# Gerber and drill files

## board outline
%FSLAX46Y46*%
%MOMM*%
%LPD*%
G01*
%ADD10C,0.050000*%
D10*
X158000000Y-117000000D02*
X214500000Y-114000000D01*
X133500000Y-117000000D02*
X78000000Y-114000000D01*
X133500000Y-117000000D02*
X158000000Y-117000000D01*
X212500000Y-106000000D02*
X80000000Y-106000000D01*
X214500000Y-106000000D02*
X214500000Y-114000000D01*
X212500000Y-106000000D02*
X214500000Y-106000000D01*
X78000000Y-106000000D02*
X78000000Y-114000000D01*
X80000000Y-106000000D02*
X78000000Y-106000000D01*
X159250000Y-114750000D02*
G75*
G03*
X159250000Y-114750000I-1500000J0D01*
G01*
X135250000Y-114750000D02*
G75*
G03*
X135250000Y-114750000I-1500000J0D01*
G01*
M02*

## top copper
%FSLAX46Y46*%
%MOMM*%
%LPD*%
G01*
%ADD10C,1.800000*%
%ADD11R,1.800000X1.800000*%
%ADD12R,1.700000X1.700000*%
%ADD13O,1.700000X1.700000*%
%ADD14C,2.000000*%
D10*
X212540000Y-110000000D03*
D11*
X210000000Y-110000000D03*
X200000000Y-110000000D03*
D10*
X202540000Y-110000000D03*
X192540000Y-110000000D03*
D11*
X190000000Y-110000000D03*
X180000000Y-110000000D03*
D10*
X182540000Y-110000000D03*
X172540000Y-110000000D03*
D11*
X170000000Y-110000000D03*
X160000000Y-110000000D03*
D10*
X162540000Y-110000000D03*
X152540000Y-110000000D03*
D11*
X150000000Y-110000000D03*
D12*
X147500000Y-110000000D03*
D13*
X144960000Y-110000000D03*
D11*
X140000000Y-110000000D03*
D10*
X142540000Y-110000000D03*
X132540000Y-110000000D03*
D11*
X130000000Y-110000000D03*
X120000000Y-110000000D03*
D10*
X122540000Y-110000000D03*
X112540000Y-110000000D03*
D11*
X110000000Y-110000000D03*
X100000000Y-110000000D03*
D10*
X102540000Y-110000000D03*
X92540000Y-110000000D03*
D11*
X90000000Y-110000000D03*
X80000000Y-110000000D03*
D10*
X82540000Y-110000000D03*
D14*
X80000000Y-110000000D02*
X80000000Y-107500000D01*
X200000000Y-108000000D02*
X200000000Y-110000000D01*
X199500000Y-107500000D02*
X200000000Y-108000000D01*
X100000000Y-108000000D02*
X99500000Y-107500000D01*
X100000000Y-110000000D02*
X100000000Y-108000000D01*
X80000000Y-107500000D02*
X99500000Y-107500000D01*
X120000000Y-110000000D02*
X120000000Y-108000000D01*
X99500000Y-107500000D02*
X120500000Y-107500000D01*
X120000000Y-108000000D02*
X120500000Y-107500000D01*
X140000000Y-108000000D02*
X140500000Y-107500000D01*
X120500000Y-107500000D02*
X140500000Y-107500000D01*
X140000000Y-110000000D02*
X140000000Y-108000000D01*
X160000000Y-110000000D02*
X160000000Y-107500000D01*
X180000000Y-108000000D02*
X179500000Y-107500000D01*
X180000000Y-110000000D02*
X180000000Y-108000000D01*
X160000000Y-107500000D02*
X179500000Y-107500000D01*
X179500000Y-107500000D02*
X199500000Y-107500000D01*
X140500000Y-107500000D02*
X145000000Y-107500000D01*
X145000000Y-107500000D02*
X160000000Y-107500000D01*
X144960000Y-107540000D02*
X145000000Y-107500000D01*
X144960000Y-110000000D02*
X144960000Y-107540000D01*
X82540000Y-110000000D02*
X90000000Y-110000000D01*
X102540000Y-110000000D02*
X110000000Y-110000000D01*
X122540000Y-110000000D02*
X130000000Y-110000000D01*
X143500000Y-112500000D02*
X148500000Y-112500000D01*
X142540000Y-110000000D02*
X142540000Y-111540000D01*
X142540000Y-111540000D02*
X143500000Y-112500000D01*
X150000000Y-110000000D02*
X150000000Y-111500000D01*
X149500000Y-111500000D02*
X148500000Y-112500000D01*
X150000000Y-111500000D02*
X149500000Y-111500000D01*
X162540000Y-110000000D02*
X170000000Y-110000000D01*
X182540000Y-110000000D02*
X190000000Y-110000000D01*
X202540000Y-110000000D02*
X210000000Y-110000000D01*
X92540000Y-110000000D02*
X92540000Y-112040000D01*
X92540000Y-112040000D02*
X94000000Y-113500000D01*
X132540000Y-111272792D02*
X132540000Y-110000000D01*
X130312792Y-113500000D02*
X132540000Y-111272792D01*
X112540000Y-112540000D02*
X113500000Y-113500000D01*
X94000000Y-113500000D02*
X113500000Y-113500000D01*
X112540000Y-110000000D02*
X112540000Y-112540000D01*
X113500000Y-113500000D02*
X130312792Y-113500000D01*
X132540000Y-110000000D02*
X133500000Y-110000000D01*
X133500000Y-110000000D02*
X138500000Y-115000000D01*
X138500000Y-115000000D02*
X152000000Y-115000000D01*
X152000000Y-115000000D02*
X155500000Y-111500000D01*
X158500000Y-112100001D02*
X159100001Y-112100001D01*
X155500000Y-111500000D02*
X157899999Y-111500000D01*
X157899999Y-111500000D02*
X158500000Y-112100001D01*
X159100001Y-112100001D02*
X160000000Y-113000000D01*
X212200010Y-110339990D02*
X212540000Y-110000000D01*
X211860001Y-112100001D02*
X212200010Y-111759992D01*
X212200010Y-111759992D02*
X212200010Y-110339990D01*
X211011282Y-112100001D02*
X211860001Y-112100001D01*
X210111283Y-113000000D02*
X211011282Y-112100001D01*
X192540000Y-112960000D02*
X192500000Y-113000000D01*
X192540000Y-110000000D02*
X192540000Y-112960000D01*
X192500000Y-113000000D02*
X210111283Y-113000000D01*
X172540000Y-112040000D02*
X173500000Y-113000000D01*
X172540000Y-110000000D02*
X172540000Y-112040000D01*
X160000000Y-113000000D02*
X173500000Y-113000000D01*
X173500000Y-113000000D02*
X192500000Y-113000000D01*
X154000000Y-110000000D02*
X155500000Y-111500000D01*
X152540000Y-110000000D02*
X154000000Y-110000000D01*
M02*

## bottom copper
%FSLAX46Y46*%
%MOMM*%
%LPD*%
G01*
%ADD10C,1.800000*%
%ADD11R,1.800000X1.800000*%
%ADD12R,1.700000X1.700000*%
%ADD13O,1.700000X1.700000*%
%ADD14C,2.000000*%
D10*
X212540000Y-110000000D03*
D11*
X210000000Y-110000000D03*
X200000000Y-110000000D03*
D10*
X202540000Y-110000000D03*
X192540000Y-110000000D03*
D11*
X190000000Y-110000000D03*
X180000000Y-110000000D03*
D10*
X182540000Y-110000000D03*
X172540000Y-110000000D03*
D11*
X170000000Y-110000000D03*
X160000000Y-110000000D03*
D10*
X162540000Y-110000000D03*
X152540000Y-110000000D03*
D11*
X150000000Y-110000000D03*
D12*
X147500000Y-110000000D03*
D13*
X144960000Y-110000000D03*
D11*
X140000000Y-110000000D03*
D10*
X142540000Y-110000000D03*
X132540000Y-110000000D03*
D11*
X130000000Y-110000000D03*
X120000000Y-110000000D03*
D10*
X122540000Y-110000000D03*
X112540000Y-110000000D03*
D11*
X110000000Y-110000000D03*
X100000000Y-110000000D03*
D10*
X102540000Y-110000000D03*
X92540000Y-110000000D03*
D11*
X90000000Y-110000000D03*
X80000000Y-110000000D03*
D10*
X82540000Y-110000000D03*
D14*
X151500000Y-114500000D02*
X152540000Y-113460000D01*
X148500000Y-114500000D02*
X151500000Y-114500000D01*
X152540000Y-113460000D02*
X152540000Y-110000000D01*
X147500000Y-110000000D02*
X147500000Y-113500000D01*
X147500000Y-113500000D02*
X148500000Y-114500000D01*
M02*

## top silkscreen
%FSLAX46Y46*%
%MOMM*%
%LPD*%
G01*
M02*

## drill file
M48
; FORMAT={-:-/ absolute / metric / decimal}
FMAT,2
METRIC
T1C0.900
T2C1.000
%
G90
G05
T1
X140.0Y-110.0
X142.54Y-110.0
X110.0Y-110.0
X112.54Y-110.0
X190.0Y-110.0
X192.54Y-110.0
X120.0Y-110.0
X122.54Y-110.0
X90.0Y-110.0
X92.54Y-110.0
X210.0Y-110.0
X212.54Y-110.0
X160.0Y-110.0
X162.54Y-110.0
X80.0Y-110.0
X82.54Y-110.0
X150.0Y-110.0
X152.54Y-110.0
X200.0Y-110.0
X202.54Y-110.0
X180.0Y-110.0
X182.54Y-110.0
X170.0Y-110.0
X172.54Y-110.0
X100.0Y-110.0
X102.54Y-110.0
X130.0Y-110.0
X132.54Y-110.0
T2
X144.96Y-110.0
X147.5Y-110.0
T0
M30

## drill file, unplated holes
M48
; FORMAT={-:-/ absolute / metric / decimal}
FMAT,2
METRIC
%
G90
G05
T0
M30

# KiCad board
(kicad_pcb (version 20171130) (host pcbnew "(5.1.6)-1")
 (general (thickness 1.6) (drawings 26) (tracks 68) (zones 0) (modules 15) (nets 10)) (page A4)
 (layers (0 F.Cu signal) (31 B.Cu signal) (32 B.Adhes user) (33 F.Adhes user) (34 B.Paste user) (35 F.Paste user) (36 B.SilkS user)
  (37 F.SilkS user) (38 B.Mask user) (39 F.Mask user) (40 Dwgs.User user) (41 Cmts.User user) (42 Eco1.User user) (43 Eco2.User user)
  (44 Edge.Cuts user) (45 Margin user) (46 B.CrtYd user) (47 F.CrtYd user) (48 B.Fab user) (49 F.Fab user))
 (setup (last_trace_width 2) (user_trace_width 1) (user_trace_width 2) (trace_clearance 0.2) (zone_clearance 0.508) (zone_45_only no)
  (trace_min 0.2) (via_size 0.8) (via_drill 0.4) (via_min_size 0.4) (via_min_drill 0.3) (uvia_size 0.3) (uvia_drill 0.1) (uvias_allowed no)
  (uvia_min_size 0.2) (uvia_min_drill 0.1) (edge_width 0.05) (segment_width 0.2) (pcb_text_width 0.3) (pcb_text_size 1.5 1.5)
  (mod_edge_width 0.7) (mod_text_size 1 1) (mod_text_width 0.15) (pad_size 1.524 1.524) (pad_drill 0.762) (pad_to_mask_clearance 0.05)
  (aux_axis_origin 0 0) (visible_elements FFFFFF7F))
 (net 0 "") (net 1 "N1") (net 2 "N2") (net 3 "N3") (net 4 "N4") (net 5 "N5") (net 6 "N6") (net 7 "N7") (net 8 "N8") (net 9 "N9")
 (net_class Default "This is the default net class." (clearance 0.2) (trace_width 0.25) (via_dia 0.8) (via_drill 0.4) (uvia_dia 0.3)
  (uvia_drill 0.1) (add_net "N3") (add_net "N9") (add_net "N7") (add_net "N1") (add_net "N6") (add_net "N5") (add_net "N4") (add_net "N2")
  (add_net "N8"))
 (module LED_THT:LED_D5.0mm (layer F.Cu) (at 210 110)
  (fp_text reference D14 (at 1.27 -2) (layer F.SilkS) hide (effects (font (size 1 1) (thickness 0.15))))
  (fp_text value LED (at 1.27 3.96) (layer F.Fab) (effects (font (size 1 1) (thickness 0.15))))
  (pad 2 thru_hole circle (at 2.54 0) (size 1.8 1.8) (drill 0.9) (layers *.Cu *.Mask) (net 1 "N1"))
  (pad 1 thru_hole rect (at 0 0) (size 1.8 1.8) (drill 0.9) (layers *.Cu *.Mask) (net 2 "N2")))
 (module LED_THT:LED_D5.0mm (layer F.Cu) (at 200 110)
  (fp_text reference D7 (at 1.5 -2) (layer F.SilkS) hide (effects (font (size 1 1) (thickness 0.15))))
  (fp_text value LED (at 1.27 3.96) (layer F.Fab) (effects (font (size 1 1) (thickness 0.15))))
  (pad 1 thru_hole rect (at 0 0) (size 1.8 1.8) (drill 0.9) (layers *.Cu *.Mask) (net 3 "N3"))
  (pad 2 thru_hole circle (at 2.54 0) (size 1.8 1.8) (drill 0.9) (layers *.Cu *.Mask) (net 2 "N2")))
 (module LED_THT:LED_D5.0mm (layer F.Cu) (at 190 110)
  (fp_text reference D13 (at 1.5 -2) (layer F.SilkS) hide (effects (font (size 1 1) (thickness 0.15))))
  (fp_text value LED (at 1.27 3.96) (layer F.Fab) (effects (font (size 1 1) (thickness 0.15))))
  (pad 2 thru_hole circle (at 2.54 0) (size 1.8 1.8) (drill 0.9) (layers *.Cu *.Mask) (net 1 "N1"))
  (pad 1 thru_hole rect (at 0 0) (size 1.8 1.8) (drill 0.9) (layers *.Cu *.Mask) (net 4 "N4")))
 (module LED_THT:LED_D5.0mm (layer F.Cu) (at 180 110)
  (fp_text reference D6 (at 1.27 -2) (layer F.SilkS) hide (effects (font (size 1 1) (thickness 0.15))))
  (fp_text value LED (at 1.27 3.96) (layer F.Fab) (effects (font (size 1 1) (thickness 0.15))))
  (pad 1 thru_hole rect (at 0 0) (size 1.8 1.8) (drill 0.9) (layers *.Cu *.Mask) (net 3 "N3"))
  (pad 2 thru_hole circle (at 2.54 0) (size 1.8 1.8) (drill 0.9) (layers *.Cu *.Mask) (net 4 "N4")))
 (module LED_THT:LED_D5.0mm (layer F.Cu) (at 170 110)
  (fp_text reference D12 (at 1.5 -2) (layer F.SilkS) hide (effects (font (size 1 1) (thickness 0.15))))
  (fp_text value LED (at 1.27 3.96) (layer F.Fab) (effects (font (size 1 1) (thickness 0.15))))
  (pad 2 thru_hole circle (at 2.54 0) (size 1.8 1.8) (drill 0.9) (layers *.Cu *.Mask) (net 1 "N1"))
  (pad 1 thru_hole rect (at 0 0) (size 1.8 1.8) (drill 0.9) (layers *.Cu *.Mask) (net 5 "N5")))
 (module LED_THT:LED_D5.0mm (layer F.Cu) (at 160 110)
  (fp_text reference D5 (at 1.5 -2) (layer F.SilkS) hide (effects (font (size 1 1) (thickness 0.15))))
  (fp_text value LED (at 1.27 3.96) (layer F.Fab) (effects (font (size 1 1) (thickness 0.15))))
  (pad 1 thru_hole rect (at 0 0) (size 1.8 1.8) (drill 0.9) (layers *.Cu *.Mask) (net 3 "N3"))
  (pad 2 thru_hole circle (at 2.54 0) (size 1.8 1.8) (drill 0.9) (layers *.Cu *.Mask) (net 5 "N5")))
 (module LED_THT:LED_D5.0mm (layer F.Cu) (at 150 110)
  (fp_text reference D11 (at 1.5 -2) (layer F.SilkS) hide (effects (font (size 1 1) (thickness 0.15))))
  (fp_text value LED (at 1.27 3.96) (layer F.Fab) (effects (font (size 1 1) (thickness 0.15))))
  (pad 2 thru_hole circle (at 2.54 0) (size 1.8 1.8) (drill 0.9) (layers *.Cu *.Mask) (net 1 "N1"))
  (pad 1 thru_hole rect (at 0 0) (size 1.8 1.8) (drill 0.9) (layers *.Cu *.Mask) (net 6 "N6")))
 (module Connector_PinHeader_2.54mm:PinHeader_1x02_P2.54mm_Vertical (layer F.Cu) (at 147.5 110 270)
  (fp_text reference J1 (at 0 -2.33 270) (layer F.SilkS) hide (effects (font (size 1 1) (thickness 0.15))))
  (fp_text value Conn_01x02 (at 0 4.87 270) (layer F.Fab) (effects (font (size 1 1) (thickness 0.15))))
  (pad 1 thru_hole rect (at 0 0 270) (size 1.7 1.7) (drill 1) (layers *.Cu *.Mask) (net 1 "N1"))
  (pad 2 thru_hole oval (at 0 2.54 270) (size 1.7 1.7) (drill 1) (layers *.Cu *.Mask) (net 3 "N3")))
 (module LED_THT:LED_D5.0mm (layer F.Cu) (at 140 110)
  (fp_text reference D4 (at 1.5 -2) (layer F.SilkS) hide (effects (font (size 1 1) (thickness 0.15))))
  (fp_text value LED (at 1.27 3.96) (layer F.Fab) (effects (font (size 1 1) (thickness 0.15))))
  (pad 1 thru_hole rect (at 0 0) (size 1.8 1.8) (drill 0.9) (layers *.Cu *.Mask) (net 3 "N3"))
  (pad 2 thru_hole circle (at 2.54 0) (size 1.8 1.8) (drill 0.9) (layers *.Cu *.Mask) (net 6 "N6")))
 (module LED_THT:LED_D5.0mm (layer F.Cu) (at 130 110)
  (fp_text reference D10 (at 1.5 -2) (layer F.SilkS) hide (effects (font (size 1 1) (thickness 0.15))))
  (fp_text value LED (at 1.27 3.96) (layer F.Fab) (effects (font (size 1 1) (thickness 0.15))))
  (pad 2 thru_hole circle (at 2.54 0) (size 1.8 1.8) (drill 0.9) (layers *.Cu *.Mask) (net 1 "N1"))
  (pad 1 thru_hole rect (at 0 0) (size 1.8 1.8) (drill 0.9) (layers *.Cu *.Mask) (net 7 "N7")))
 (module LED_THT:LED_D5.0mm (layer F.Cu) (at 120 110)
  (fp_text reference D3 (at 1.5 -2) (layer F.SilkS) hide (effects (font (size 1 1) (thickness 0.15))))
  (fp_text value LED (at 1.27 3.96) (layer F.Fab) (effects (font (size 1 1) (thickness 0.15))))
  (pad 1 thru_hole rect (at 0 0) (size 1.8 1.8) (drill 0.9) (layers *.Cu *.Mask) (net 3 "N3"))
  (pad 2 thru_hole circle (at 2.54 0) (size 1.8 1.8) (drill 0.9) (layers *.Cu *.Mask) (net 7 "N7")))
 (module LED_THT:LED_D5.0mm (layer F.Cu) (at 110 110)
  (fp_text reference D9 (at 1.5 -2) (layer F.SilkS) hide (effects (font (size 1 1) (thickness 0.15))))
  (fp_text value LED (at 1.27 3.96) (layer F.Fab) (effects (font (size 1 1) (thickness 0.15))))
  (pad 2 thru_hole circle (at 2.54 0) (size 1.8 1.8) (drill 0.9) (layers *.Cu *.Mask) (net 1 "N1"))
  (pad 1 thru_hole rect (at 0 0) (size 1.8 1.8) (drill 0.9) (layers *.Cu *.Mask) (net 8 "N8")))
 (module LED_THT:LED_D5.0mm (layer F.Cu) (at 100 110)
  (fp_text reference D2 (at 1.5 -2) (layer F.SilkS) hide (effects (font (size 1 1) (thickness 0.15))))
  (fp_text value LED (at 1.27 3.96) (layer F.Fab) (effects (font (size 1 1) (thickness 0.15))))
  (pad 1 thru_hole rect (at 0 0) (size 1.8 1.8) (drill 0.9) (layers *.Cu *.Mask) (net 3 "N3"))
  (pad 2 thru_hole circle (at 2.54 0) (size 1.8 1.8) (drill 0.9) (layers *.Cu *.Mask) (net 8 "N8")))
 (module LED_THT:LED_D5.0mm (layer F.Cu) (at 90 110)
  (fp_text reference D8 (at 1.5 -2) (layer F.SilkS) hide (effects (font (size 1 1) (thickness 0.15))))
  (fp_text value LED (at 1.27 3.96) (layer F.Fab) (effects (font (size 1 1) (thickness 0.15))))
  (pad 2 thru_hole circle (at 2.54 0) (size 1.8 1.8) (drill 0.9) (layers *.Cu *.Mask) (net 1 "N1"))
  (pad 1 thru_hole rect (at 0 0) (size 1.8 1.8) (drill 0.9) (layers *.Cu *.Mask) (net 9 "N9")))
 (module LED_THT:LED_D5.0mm (layer F.Cu) (at 80 110)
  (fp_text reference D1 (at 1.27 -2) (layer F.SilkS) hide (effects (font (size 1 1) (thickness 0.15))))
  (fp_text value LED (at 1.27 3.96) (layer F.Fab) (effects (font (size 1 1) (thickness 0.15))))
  (pad 1 thru_hole rect (at 0 0) (size 1.8 1.8) (drill 0.9) (layers *.Cu *.Mask) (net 3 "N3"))
  (pad 2 thru_hole circle (at 2.54 0) (size 1.8 1.8) (drill 0.9) (layers *.Cu *.Mask) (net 9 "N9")))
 (gr_line (start 158 117) (end 214.5 114) (layer Edge.Cuts) (width 0.05))
 (gr_line (start 133.5 117) (end 78 114) (layer Edge.Cuts) (width 0.05))
 (gr_line (start 133.5 117) (end 158 117) (layer Edge.Cuts) (width 0.05))
 (gr_line (start 212.5 106) (end 80 106) (layer Edge.Cuts) (width 0.05))
 (gr_line (start 214.5 106) (end 214.5 114) (layer Edge.Cuts) (width 0.05))
 (gr_line (start 212.5 106) (end 214.5 106) (layer Edge.Cuts) (width 0.05))
 (gr_line (start 78 106) (end 78 114) (layer Edge.Cuts) (width 0.05))
 (gr_line (start 80 106) (end 78 106) (layer Edge.Cuts) (width 0.05))
 (gr_circle (center 157.75 114.75) (end 159.25 114.75) (layer Edge.Cuts) (width 0.05))
 (gr_circle (center 133.75 114.75) (end 132.25 114.75) (layer Edge.Cuts) (width 0.05))
 (segment (start 80 110) (end 80 107.5) (width 2) (layer F.Cu) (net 3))
 (segment (start 200 108) (end 200 110) (width 2) (layer F.Cu) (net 3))
 (segment (start 199.5 107.5) (end 200 108) (width 2) (layer F.Cu) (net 3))
 (segment (start 100 108) (end 99.5 107.5) (width 2) (layer F.Cu) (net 3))
 (segment (start 100 110) (end 100 108) (width 2) (layer F.Cu) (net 3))
 (segment (start 80 107.5) (end 99.5 107.5) (width 2) (layer F.Cu) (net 3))
 (segment (start 120 110) (end 120 108) (width 2) (layer F.Cu) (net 3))
 (segment (start 99.5 107.5) (end 120.5 107.5) (width 2) (layer F.Cu) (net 3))
 (segment (start 120 108) (end 120.5 107.5) (width 2) (layer F.Cu) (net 3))
 (segment (start 140 108) (end 140.5 107.5) (width 2) (layer F.Cu) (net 3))
 (segment (start 120.5 107.5) (end 140.5 107.5) (width 2) (layer F.Cu) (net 3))
 (segment (start 140 110) (end 140 108) (width 2) (layer F.Cu) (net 3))
 (segment (start 160 110) (end 160 107.5) (width 2) (layer F.Cu) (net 3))
 (segment (start 180 108) (end 179.5 107.5) (width 2) (layer F.Cu) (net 3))
 (segment (start 180 110) (end 180 108) (width 2) (layer F.Cu) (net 3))
 (segment (start 160 107.5) (end 179.5 107.5) (width 2) (layer F.Cu) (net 3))
 (segment (start 179.5 107.5) (end 199.5 107.5) (width 2) (layer F.Cu) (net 3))
 (segment (start 140.5 107.5) (end 145 107.5) (width 2) (layer F.Cu) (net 3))
 (segment (start 145 107.5) (end 160 107.5) (width 2) (layer F.Cu) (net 3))
 (segment (start 144.96 107.54) (end 145 107.5) (width 2) (layer F.Cu) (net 3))
 (segment (start 144.96 110) (end 144.96 107.54) (width 2) (layer F.Cu) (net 3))
 (segment (start 82.54 110) (end 90 110) (width 2) (layer F.Cu) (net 9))
 (segment (start 102.54 110) (end 110 110) (width 2) (layer F.Cu) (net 8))
 (segment (start 122.54 110) (end 130 110) (width 2) (layer F.Cu) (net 7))
 (segment (start 143.5 112.5) (end 148.5 112.5) (width 2) (layer F.Cu) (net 6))
 (segment (start 142.54 110) (end 142.54 111.54) (width 2) (layer F.Cu) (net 6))
 (segment (start 142.54 111.54) (end 143.5 112.5) (width 2) (layer F.Cu) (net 6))
 (segment (start 150 110) (end 150 111.5) (width 2) (layer F.Cu) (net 6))
 (segment (start 149.5 111.5) (end 148.5 112.5) (width 2) (layer F.Cu) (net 6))
 (segment (start 150 111.5) (end 149.5 111.5) (width 2) (layer F.Cu) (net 6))
 (segment (start 162.54 110) (end 170 110) (width 2) (layer F.Cu) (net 5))
 (segment (start 182.54 110) (end 190 110) (width 2) (layer F.Cu) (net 4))
 (segment (start 202.54 110) (end 210 110) (width 2) (layer F.Cu) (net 2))
 (segment (start 92.54 110) (end 92.54 112.04) (width 2) (layer F.Cu) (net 1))
 (segment (start 92.54 112.04) (end 94 113.5) (width 2) (layer F.Cu) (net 1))
 (segment (start 132.54 111.272792) (end 132.54 110) (width 2) (layer F.Cu) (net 1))
 (segment (start 130.312792 113.5) (end 132.54 111.272792) (width 2) (layer F.Cu) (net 1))
 (segment (start 112.54 112.54) (end 113.5 113.5) (width 2) (layer F.Cu) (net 1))
 (segment (start 94 113.5) (end 113.5 113.5) (width 2) (layer F.Cu) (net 1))
 (segment (start 112.54 110) (end 112.54 112.54) (width 2) (layer F.Cu) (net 1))
 (segment (start 113.5 113.5) (end 130.312792 113.5) (width 2) (layer F.Cu) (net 1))
 (segment (start 132.54 110) (end 133.5 110) (width 2) (layer F.Cu) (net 1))
 (segment (start 133.5 110) (end 138.5 115) (width 2) (layer F.Cu) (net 1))
 (segment (start 138.5 115) (end 152 115) (width 2) (layer F.Cu) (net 1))
 (segment (start 152 115) (end 155.5 111.5) (width 2) (layer F.Cu) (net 1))
 (segment (start 158.5 112.100001) (end 159.100001 112.100001) (width 2) (layer F.Cu) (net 1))
 (segment (start 155.5 111.5) (end 157.899999 111.5) (width 2) (layer F.Cu) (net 1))
 (segment (start 157.899999 111.5) (end 158.5 112.100001) (width 2) (layer F.Cu) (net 1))
 (segment (start 159.100001 112.100001) (end 160 113) (width 2) (layer F.Cu) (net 1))
 (segment (start 212.20001 110.33999) (end 212.54 110) (width 2) (layer F.Cu) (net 1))
 (segment (start 211.860001 112.100001) (end 212.20001 111.759992) (width 2) (layer F.Cu) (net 1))
 (segment (start 212.20001 111.759992) (end 212.20001 110.33999) (width 2) (layer F.Cu) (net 1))
 (segment (start 211.011282 112.100001) (end 211.860001 112.100001) (width 2) (layer F.Cu) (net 1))
 (segment (start 210.111283 113) (end 211.011282 112.100001) (width 2) (layer F.Cu) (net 1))
 (segment (start 192.54 112.96) (end 192.5 113) (width 2) (layer F.Cu) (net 1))
 (segment (start 192.54 110) (end 192.54 112.96) (width 2) (layer F.Cu) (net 1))
 (segment (start 192.5 113) (end 210.111283 113) (width 2) (layer F.Cu) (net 1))
 (segment (start 172.54 112.04) (end 173.5 113) (width 2) (layer F.Cu) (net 1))
 (segment (start 172.54 110) (end 172.54 112.04) (width 2) (layer F.Cu) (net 1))
 (segment (start 160 113) (end 173.5 113) (width 2) (layer F.Cu) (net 1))
 (segment (start 173.5 113) (end 192.5 113) (width 2) (layer F.Cu) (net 1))
 (segment (start 154 110) (end 155.5 111.5) (width 2) (layer F.Cu) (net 1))
 (segment (start 152.54 110) (end 154 110) (width 2) (layer F.Cu) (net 1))
 (segment (start 151.5 114.5) (end 152.54 113.46) (width 2) (layer B.Cu) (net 1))
 (segment (start 148.5 114.5) (end 151.5 114.5) (width 2) (layer B.Cu) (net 1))
 (segment (start 152.54 113.46) (end 152.54 110) (width 2) (layer B.Cu) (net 1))
 (segment (start 147.5 110) (end 147.5 113.5) (width 2) (layer B.Cu) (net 1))
 (segment (start 147.5 113.5) (end 148.5 114.5) (width 2) (layer B.Cu) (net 1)))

